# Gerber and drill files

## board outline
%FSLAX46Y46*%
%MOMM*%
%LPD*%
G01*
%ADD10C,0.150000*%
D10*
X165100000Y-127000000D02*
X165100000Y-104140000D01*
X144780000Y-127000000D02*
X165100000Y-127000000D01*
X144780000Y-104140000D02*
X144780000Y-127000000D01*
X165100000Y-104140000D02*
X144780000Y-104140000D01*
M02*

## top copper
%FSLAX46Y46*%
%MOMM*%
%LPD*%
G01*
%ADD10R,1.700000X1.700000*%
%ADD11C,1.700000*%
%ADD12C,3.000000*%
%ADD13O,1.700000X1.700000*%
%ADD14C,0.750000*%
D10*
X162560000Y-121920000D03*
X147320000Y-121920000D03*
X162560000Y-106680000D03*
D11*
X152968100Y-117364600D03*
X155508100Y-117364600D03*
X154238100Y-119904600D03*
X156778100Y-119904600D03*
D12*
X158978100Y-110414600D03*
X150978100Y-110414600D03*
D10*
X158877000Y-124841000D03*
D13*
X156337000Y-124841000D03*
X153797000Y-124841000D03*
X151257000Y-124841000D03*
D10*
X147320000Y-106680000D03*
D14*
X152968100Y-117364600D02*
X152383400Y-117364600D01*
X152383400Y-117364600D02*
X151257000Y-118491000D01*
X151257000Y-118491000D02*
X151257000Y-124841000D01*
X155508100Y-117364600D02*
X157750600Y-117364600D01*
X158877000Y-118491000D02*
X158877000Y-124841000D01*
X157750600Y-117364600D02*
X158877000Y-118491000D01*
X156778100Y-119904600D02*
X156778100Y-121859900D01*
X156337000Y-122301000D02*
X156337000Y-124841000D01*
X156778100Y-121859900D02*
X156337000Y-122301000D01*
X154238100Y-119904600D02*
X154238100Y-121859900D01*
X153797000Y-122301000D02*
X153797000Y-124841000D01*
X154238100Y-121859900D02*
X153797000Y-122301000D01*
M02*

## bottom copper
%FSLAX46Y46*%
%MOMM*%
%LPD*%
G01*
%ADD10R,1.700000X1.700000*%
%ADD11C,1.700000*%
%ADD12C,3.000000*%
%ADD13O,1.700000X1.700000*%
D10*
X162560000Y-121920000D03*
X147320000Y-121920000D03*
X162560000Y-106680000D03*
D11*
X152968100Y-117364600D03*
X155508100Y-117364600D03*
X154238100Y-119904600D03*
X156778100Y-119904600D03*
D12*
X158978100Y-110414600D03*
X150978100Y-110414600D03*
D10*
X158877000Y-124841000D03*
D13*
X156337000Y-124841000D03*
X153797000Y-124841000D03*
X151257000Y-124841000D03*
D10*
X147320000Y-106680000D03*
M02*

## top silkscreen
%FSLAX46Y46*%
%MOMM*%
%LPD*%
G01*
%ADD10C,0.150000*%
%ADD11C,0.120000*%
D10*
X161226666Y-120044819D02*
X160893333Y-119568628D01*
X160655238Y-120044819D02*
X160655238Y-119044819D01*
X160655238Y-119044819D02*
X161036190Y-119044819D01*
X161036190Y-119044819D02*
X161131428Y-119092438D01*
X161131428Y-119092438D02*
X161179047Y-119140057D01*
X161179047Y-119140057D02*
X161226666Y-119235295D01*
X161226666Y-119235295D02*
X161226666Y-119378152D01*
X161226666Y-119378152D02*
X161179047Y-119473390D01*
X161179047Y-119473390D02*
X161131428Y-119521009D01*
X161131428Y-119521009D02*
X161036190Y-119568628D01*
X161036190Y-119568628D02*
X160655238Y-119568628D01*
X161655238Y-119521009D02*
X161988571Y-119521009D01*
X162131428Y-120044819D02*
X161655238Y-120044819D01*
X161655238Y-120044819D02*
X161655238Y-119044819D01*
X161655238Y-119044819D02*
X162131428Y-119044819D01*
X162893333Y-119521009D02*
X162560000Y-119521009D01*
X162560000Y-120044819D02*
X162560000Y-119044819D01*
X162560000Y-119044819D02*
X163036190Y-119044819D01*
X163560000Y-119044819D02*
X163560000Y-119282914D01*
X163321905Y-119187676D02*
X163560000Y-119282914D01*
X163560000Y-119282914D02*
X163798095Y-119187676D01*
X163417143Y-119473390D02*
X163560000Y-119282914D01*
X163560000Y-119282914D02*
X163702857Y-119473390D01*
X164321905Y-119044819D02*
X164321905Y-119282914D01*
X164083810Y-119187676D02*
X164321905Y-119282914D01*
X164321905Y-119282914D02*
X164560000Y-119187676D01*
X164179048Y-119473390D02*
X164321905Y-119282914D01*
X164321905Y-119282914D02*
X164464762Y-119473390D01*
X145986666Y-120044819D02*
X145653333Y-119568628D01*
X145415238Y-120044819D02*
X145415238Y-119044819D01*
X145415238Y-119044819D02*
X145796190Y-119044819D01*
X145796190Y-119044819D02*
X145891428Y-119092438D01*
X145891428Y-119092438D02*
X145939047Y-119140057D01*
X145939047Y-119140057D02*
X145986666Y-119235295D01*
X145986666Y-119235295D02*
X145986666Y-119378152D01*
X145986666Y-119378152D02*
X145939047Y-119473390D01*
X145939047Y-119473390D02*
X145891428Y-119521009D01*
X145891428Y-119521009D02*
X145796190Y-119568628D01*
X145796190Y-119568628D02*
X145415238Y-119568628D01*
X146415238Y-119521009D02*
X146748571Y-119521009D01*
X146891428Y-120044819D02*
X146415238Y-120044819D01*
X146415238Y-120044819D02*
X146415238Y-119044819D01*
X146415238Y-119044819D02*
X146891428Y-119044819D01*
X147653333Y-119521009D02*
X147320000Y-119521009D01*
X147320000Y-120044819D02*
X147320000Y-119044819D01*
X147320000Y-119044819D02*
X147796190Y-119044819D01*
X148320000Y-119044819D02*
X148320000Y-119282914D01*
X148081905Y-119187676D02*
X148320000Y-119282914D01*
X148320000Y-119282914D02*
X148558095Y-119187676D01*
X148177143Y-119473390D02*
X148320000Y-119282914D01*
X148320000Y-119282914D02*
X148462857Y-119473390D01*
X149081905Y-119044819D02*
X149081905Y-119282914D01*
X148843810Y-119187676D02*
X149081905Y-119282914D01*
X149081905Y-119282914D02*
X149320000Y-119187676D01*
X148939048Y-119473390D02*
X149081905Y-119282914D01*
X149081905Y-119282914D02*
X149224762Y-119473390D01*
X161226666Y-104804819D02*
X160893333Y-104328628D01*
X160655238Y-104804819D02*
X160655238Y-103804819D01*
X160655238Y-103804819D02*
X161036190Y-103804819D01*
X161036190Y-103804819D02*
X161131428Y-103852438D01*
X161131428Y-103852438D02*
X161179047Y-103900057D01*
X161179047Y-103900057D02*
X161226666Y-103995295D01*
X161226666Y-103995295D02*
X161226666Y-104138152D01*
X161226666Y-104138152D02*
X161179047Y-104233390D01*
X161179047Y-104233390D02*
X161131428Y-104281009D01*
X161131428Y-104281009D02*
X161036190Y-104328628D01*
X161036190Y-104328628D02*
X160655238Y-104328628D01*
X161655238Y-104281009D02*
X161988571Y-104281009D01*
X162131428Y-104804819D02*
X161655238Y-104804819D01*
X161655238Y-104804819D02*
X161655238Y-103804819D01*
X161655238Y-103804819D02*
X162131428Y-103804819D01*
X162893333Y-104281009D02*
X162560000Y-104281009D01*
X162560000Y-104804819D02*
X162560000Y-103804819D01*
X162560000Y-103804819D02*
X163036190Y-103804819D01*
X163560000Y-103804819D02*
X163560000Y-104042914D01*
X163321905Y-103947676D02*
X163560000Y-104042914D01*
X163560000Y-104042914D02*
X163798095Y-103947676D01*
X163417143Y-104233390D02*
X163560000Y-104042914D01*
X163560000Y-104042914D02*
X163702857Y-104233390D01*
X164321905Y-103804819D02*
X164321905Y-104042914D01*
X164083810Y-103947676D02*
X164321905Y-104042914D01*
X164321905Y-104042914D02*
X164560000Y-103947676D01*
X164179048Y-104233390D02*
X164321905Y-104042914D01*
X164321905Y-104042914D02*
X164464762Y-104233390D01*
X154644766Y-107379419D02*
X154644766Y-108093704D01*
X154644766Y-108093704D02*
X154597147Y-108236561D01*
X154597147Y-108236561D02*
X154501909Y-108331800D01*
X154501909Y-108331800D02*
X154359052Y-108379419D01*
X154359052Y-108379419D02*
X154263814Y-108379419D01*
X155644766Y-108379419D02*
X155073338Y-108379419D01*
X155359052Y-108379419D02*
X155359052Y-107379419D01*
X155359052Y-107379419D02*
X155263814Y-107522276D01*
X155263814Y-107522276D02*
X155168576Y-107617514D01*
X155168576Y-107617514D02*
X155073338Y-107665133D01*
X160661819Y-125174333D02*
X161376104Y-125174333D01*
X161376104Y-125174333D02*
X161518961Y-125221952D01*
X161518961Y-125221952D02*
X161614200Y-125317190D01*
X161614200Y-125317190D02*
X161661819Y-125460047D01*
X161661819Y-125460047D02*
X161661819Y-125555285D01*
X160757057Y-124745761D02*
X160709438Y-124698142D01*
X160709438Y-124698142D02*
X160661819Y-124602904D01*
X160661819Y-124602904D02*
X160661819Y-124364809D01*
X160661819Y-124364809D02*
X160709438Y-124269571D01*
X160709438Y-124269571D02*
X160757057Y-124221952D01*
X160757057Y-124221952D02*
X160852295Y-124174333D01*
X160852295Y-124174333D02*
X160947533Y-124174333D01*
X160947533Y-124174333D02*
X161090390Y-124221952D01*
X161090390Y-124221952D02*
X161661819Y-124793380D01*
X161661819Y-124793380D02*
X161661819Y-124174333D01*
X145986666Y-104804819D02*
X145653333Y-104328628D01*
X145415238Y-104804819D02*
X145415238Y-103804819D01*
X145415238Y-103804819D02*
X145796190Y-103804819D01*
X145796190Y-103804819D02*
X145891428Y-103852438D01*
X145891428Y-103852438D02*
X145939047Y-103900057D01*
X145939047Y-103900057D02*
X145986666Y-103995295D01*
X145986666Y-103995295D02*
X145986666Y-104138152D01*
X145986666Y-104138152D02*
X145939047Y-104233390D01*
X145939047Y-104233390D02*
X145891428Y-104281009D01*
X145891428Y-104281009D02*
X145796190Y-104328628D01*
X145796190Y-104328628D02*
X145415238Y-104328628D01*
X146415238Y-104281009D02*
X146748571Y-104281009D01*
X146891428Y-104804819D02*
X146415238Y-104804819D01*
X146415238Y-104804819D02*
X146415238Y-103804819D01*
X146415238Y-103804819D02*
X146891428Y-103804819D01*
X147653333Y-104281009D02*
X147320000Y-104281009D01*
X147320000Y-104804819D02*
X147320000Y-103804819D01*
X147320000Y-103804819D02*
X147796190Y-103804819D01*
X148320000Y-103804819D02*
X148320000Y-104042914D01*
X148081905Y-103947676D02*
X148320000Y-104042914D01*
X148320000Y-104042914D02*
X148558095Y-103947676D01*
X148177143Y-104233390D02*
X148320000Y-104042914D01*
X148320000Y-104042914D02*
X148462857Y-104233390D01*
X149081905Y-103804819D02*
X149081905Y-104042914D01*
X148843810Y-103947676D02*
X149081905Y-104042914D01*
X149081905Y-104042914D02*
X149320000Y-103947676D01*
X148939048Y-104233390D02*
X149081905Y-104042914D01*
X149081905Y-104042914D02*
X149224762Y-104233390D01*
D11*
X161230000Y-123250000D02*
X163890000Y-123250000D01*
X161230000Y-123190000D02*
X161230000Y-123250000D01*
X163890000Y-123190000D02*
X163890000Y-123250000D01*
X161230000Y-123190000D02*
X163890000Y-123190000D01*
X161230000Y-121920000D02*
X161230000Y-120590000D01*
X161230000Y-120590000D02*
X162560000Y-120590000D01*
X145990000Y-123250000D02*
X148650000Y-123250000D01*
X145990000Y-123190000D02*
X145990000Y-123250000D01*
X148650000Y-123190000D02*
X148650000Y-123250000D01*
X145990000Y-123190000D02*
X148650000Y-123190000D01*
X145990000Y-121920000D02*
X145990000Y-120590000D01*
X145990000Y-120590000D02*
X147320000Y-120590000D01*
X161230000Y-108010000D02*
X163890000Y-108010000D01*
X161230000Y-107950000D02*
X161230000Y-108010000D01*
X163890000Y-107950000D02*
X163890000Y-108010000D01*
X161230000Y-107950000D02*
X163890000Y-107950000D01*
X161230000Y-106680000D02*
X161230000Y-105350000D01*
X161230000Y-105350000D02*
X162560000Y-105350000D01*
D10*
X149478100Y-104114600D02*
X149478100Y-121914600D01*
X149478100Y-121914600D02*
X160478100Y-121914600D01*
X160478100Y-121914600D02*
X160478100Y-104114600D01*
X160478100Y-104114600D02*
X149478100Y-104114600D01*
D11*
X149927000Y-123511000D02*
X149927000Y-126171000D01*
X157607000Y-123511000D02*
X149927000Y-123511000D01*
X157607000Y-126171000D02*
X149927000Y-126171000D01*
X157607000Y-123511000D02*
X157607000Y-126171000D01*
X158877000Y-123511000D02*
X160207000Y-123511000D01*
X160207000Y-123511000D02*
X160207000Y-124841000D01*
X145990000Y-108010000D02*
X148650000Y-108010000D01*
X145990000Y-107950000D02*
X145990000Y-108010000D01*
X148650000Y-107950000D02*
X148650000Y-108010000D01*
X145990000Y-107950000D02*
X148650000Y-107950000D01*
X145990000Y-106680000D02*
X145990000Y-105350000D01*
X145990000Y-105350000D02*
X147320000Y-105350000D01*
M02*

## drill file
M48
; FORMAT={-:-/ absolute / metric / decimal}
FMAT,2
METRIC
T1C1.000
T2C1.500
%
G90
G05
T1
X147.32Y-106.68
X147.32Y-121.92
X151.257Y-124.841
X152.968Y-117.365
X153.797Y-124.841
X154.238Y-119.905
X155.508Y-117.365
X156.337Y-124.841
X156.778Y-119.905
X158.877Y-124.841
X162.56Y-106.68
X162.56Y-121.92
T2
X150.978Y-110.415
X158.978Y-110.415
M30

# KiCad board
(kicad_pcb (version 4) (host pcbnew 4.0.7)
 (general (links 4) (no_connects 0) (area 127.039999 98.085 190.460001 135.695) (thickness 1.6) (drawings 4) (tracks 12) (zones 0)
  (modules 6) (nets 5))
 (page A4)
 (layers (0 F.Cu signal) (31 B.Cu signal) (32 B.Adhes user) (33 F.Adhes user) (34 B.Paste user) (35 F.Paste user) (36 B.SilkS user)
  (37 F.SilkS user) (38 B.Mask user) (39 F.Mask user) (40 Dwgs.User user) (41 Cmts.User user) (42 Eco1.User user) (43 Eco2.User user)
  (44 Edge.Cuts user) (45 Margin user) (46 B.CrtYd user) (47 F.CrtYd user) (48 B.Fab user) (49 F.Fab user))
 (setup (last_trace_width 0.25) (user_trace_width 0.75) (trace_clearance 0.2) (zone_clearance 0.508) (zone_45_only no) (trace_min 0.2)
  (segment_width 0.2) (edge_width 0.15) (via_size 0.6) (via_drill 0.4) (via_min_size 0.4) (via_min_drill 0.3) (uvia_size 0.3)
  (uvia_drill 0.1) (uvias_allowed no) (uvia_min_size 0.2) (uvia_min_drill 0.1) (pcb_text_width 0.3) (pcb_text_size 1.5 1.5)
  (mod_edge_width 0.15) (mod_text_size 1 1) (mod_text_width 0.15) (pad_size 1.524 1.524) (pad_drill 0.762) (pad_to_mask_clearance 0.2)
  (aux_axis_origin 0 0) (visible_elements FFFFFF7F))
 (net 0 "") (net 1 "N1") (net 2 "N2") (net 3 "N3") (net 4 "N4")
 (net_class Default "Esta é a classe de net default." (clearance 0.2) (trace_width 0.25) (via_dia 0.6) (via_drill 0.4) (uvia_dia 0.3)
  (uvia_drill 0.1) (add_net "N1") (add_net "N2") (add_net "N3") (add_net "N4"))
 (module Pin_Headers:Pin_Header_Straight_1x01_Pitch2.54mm (layer F.Cu) (at 162.56 121.92)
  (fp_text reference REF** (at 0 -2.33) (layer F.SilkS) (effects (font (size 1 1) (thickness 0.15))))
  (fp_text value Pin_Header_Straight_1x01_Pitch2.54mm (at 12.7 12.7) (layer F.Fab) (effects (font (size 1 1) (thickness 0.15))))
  (fp_line (start -1.33 1.33) (end 1.33 1.33) (layer F.SilkS) (width 0.12))
  (fp_line (start -1.33 1.27) (end -1.33 1.33) (layer F.SilkS) (width 0.12))
  (fp_line (start 1.33 1.27) (end 1.33 1.33) (layer F.SilkS) (width 0.12))
  (fp_line (start -1.33 1.27) (end 1.33 1.27) (layer F.SilkS) (width 0.12))
  (fp_line (start -1.33 0) (end -1.33 -1.33) (layer F.SilkS) (width 0.12))
  (fp_line (start -1.33 -1.33) (end 0 -1.33) (layer F.SilkS) (width 0.12))
  (pad 1 thru_hole rect (at 0 0) (size 1.7 1.7) (drill 1) (layers *.Cu *.Mask)))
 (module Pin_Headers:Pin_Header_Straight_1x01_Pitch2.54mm (layer F.Cu) (at 147.32 121.92)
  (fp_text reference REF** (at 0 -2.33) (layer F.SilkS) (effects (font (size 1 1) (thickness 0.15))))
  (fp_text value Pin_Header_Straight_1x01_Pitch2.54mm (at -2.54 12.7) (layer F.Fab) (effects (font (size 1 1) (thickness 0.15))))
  (fp_line (start -1.33 1.33) (end 1.33 1.33) (layer F.SilkS) (width 0.12))
  (fp_line (start -1.33 1.27) (end -1.33 1.33) (layer F.SilkS) (width 0.12))
  (fp_line (start 1.33 1.27) (end 1.33 1.33) (layer F.SilkS) (width 0.12))
  (fp_line (start -1.33 1.27) (end 1.33 1.27) (layer F.SilkS) (width 0.12))
  (fp_line (start -1.33 0) (end -1.33 -1.33) (layer F.SilkS) (width 0.12))
  (fp_line (start -1.33 -1.33) (end 0 -1.33) (layer F.SilkS) (width 0.12))
  (pad 1 thru_hole rect (at 0 0) (size 1.7 1.7) (drill 1) (layers *.Cu *.Mask)))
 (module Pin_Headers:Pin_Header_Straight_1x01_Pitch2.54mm (layer F.Cu) (at 162.56 106.68)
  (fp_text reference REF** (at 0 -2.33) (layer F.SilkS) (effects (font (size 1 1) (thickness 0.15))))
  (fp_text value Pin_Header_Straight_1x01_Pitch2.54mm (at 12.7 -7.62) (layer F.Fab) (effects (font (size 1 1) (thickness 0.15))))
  (fp_line (start -1.33 1.33) (end 1.33 1.33) (layer F.SilkS) (width 0.12))
  (fp_line (start -1.33 1.27) (end -1.33 1.33) (layer F.SilkS) (width 0.12))
  (fp_line (start 1.33 1.27) (end 1.33 1.33) (layer F.SilkS) (width 0.12))
  (fp_line (start -1.33 1.27) (end 1.33 1.27) (layer F.SilkS) (width 0.12))
  (fp_line (start -1.33 0) (end -1.33 -1.33) (layer F.SilkS) (width 0.12))
  (fp_line (start -1.33 -1.33) (end 0 -1.33) (layer F.SilkS) (width 0.12))
  (pad 1 thru_hole rect (at 0 0) (size 1.7 1.7) (drill 1) (layers *.Cu *.Mask)))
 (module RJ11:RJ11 (layer F.Cu) (at 154.9781 104.1146)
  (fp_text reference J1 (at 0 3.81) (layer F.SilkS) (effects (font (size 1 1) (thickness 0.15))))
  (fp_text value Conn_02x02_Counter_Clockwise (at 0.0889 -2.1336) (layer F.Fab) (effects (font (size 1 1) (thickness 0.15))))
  (fp_line (start -5.5 0) (end -5.5 17.8) (layer F.SilkS) (width 0.15))
  (fp_line (start -5.5 17.8) (end 5.5 17.8) (layer F.SilkS) (width 0.15))
  (fp_line (start 5.5 17.8) (end 5.5 0) (layer F.SilkS) (width 0.15))
  (fp_line (start 5.5 0) (end -5.5 0) (layer F.SilkS) (width 0.15))
  (pad 1 thru_hole circle (at -2.01 13.25) (size 1.7 1.7) (drill 1) (layers *.Cu *.Mask) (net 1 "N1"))
  (pad 2 thru_hole circle (at 0.53 13.25) (size 1.7 1.7) (drill 1) (layers *.Cu *.Mask) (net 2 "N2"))
  (pad 3 thru_hole circle (at -0.74 15.79) (size 1.7 1.7) (drill 1) (layers *.Cu *.Mask) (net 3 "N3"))
  (pad 4 thru_hole circle (at 1.8 15.79) (size 1.7 1.7) (drill 1) (layers *.Cu *.Mask) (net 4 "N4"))
  (pad 6 thru_hole circle (at 4 6.3) (size 3 3) (drill 1.5) (layers *.Cu *.Mask))
  (pad 5 thru_hole circle (at -4 6.3) (size 3 3) (drill 1.5) (layers *.Cu *.Mask)))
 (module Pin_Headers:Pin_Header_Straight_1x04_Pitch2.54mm (layer F.Cu) (at 158.877 124.841 270)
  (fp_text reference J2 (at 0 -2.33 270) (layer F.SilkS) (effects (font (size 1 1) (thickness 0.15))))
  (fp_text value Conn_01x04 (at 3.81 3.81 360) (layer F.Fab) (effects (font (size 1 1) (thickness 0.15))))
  (fp_line (start -1.33 8.95) (end 1.33 8.95) (layer F.SilkS) (width 0.12))
  (fp_line (start -1.33 1.27) (end -1.33 8.95) (layer F.SilkS) (width 0.12))
  (fp_line (start 1.33 1.27) (end 1.33 8.95) (layer F.SilkS) (width 0.12))
  (fp_line (start -1.33 1.27) (end 1.33 1.27) (layer F.SilkS) (width 0.12))
  (fp_line (start -1.33 0) (end -1.33 -1.33) (layer F.SilkS) (width 0.12))
  (fp_line (start -1.33 -1.33) (end 0 -1.33) (layer F.SilkS) (width 0.12))
  (pad 1 thru_hole rect (at 0 0 270) (size 1.7 1.7) (drill 1) (layers *.Cu *.Mask) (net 2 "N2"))
  (pad 2 thru_hole oval (at 0 2.54 270) (size 1.7 1.7) (drill 1) (layers *.Cu *.Mask) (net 4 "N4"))
  (pad 3 thru_hole oval (at 0 5.08 270) (size 1.7 1.7) (drill 1) (layers *.Cu *.Mask) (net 3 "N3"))
  (pad 4 thru_hole oval (at 0 7.62 270) (size 1.7 1.7) (drill 1) (layers *.Cu *.Mask) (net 1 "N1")))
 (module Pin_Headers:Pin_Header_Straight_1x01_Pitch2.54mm (layer F.Cu) (at 147.32 106.68)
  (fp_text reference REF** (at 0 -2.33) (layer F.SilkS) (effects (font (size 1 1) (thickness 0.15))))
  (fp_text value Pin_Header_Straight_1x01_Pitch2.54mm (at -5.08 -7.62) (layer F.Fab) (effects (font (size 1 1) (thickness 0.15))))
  (fp_line (start -1.33 1.33) (end 1.33 1.33) (layer F.SilkS) (width 0.12))
  (fp_line (start -1.33 1.27) (end -1.33 1.33) (layer F.SilkS) (width 0.12))
  (fp_line (start 1.33 1.27) (end 1.33 1.33) (layer F.SilkS) (width 0.12))
  (fp_line (start -1.33 1.27) (end 1.33 1.27) (layer F.SilkS) (width 0.12))
  (fp_line (start -1.33 0) (end -1.33 -1.33) (layer F.SilkS) (width 0.12))
  (fp_line (start -1.33 -1.33) (end 0 -1.33) (layer F.SilkS) (width 0.12))
  (pad 1 thru_hole rect (at 0 0) (size 1.7 1.7) (drill 1) (layers *.Cu *.Mask)))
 (gr_line (start 165.1 127) (end 165.1 104.14) (angle 90) (layer Edge.Cuts) (width 0.15))
 (gr_line (start 144.78 127) (end 165.1 127) (angle 90) (layer Edge.Cuts) (width 0.15))
 (gr_line (start 144.78 104.14) (end 144.78 127) (angle 90) (layer Edge.Cuts) (width 0.15))
 (gr_line (start 165.1 104.14) (end 144.78 104.14) (angle 90) (layer Edge.Cuts) (width 0.15))
 (segment (start 152.9681 117.3646) (end 152.3834 117.3646) (width 0.75) (layer F.Cu) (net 1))
 (segment (start 152.3834 117.3646) (end 151.257 118.491) (width 0.75) (layer F.Cu) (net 1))
 (segment (start 151.257 118.491) (end 151.257 124.841) (width 0.75) (layer F.Cu) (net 1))
 (segment (start 155.5081 117.3646) (end 157.7506 117.3646) (width 0.75) (layer F.Cu) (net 2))
 (segment (start 158.877 118.491) (end 158.877 124.841) (width 0.75) (layer F.Cu) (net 2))
 (segment (start 157.7506 117.3646) (end 158.877 118.491) (width 0.75) (layer F.Cu) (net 2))
 (segment (start 156.7781 119.9046) (end 156.7781 121.8599) (width 0.75) (layer F.Cu) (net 4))
 (segment (start 156.337 122.301) (end 156.337 124.841) (width 0.75) (layer F.Cu) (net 4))
 (segment (start 156.7781 121.8599) (end 156.337 122.301) (width 0.75) (layer F.Cu) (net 4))
 (segment (start 154.2381 119.9046) (end 154.2381 121.8599) (width 0.75) (layer F.Cu) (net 3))
 (segment (start 153.797 122.301) (end 153.797 124.841) (width 0.75) (layer F.Cu) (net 3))
 (segment (start 154.2381 121.8599) (end 153.797 122.301) (width 0.75) (layer F.Cu) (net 3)))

